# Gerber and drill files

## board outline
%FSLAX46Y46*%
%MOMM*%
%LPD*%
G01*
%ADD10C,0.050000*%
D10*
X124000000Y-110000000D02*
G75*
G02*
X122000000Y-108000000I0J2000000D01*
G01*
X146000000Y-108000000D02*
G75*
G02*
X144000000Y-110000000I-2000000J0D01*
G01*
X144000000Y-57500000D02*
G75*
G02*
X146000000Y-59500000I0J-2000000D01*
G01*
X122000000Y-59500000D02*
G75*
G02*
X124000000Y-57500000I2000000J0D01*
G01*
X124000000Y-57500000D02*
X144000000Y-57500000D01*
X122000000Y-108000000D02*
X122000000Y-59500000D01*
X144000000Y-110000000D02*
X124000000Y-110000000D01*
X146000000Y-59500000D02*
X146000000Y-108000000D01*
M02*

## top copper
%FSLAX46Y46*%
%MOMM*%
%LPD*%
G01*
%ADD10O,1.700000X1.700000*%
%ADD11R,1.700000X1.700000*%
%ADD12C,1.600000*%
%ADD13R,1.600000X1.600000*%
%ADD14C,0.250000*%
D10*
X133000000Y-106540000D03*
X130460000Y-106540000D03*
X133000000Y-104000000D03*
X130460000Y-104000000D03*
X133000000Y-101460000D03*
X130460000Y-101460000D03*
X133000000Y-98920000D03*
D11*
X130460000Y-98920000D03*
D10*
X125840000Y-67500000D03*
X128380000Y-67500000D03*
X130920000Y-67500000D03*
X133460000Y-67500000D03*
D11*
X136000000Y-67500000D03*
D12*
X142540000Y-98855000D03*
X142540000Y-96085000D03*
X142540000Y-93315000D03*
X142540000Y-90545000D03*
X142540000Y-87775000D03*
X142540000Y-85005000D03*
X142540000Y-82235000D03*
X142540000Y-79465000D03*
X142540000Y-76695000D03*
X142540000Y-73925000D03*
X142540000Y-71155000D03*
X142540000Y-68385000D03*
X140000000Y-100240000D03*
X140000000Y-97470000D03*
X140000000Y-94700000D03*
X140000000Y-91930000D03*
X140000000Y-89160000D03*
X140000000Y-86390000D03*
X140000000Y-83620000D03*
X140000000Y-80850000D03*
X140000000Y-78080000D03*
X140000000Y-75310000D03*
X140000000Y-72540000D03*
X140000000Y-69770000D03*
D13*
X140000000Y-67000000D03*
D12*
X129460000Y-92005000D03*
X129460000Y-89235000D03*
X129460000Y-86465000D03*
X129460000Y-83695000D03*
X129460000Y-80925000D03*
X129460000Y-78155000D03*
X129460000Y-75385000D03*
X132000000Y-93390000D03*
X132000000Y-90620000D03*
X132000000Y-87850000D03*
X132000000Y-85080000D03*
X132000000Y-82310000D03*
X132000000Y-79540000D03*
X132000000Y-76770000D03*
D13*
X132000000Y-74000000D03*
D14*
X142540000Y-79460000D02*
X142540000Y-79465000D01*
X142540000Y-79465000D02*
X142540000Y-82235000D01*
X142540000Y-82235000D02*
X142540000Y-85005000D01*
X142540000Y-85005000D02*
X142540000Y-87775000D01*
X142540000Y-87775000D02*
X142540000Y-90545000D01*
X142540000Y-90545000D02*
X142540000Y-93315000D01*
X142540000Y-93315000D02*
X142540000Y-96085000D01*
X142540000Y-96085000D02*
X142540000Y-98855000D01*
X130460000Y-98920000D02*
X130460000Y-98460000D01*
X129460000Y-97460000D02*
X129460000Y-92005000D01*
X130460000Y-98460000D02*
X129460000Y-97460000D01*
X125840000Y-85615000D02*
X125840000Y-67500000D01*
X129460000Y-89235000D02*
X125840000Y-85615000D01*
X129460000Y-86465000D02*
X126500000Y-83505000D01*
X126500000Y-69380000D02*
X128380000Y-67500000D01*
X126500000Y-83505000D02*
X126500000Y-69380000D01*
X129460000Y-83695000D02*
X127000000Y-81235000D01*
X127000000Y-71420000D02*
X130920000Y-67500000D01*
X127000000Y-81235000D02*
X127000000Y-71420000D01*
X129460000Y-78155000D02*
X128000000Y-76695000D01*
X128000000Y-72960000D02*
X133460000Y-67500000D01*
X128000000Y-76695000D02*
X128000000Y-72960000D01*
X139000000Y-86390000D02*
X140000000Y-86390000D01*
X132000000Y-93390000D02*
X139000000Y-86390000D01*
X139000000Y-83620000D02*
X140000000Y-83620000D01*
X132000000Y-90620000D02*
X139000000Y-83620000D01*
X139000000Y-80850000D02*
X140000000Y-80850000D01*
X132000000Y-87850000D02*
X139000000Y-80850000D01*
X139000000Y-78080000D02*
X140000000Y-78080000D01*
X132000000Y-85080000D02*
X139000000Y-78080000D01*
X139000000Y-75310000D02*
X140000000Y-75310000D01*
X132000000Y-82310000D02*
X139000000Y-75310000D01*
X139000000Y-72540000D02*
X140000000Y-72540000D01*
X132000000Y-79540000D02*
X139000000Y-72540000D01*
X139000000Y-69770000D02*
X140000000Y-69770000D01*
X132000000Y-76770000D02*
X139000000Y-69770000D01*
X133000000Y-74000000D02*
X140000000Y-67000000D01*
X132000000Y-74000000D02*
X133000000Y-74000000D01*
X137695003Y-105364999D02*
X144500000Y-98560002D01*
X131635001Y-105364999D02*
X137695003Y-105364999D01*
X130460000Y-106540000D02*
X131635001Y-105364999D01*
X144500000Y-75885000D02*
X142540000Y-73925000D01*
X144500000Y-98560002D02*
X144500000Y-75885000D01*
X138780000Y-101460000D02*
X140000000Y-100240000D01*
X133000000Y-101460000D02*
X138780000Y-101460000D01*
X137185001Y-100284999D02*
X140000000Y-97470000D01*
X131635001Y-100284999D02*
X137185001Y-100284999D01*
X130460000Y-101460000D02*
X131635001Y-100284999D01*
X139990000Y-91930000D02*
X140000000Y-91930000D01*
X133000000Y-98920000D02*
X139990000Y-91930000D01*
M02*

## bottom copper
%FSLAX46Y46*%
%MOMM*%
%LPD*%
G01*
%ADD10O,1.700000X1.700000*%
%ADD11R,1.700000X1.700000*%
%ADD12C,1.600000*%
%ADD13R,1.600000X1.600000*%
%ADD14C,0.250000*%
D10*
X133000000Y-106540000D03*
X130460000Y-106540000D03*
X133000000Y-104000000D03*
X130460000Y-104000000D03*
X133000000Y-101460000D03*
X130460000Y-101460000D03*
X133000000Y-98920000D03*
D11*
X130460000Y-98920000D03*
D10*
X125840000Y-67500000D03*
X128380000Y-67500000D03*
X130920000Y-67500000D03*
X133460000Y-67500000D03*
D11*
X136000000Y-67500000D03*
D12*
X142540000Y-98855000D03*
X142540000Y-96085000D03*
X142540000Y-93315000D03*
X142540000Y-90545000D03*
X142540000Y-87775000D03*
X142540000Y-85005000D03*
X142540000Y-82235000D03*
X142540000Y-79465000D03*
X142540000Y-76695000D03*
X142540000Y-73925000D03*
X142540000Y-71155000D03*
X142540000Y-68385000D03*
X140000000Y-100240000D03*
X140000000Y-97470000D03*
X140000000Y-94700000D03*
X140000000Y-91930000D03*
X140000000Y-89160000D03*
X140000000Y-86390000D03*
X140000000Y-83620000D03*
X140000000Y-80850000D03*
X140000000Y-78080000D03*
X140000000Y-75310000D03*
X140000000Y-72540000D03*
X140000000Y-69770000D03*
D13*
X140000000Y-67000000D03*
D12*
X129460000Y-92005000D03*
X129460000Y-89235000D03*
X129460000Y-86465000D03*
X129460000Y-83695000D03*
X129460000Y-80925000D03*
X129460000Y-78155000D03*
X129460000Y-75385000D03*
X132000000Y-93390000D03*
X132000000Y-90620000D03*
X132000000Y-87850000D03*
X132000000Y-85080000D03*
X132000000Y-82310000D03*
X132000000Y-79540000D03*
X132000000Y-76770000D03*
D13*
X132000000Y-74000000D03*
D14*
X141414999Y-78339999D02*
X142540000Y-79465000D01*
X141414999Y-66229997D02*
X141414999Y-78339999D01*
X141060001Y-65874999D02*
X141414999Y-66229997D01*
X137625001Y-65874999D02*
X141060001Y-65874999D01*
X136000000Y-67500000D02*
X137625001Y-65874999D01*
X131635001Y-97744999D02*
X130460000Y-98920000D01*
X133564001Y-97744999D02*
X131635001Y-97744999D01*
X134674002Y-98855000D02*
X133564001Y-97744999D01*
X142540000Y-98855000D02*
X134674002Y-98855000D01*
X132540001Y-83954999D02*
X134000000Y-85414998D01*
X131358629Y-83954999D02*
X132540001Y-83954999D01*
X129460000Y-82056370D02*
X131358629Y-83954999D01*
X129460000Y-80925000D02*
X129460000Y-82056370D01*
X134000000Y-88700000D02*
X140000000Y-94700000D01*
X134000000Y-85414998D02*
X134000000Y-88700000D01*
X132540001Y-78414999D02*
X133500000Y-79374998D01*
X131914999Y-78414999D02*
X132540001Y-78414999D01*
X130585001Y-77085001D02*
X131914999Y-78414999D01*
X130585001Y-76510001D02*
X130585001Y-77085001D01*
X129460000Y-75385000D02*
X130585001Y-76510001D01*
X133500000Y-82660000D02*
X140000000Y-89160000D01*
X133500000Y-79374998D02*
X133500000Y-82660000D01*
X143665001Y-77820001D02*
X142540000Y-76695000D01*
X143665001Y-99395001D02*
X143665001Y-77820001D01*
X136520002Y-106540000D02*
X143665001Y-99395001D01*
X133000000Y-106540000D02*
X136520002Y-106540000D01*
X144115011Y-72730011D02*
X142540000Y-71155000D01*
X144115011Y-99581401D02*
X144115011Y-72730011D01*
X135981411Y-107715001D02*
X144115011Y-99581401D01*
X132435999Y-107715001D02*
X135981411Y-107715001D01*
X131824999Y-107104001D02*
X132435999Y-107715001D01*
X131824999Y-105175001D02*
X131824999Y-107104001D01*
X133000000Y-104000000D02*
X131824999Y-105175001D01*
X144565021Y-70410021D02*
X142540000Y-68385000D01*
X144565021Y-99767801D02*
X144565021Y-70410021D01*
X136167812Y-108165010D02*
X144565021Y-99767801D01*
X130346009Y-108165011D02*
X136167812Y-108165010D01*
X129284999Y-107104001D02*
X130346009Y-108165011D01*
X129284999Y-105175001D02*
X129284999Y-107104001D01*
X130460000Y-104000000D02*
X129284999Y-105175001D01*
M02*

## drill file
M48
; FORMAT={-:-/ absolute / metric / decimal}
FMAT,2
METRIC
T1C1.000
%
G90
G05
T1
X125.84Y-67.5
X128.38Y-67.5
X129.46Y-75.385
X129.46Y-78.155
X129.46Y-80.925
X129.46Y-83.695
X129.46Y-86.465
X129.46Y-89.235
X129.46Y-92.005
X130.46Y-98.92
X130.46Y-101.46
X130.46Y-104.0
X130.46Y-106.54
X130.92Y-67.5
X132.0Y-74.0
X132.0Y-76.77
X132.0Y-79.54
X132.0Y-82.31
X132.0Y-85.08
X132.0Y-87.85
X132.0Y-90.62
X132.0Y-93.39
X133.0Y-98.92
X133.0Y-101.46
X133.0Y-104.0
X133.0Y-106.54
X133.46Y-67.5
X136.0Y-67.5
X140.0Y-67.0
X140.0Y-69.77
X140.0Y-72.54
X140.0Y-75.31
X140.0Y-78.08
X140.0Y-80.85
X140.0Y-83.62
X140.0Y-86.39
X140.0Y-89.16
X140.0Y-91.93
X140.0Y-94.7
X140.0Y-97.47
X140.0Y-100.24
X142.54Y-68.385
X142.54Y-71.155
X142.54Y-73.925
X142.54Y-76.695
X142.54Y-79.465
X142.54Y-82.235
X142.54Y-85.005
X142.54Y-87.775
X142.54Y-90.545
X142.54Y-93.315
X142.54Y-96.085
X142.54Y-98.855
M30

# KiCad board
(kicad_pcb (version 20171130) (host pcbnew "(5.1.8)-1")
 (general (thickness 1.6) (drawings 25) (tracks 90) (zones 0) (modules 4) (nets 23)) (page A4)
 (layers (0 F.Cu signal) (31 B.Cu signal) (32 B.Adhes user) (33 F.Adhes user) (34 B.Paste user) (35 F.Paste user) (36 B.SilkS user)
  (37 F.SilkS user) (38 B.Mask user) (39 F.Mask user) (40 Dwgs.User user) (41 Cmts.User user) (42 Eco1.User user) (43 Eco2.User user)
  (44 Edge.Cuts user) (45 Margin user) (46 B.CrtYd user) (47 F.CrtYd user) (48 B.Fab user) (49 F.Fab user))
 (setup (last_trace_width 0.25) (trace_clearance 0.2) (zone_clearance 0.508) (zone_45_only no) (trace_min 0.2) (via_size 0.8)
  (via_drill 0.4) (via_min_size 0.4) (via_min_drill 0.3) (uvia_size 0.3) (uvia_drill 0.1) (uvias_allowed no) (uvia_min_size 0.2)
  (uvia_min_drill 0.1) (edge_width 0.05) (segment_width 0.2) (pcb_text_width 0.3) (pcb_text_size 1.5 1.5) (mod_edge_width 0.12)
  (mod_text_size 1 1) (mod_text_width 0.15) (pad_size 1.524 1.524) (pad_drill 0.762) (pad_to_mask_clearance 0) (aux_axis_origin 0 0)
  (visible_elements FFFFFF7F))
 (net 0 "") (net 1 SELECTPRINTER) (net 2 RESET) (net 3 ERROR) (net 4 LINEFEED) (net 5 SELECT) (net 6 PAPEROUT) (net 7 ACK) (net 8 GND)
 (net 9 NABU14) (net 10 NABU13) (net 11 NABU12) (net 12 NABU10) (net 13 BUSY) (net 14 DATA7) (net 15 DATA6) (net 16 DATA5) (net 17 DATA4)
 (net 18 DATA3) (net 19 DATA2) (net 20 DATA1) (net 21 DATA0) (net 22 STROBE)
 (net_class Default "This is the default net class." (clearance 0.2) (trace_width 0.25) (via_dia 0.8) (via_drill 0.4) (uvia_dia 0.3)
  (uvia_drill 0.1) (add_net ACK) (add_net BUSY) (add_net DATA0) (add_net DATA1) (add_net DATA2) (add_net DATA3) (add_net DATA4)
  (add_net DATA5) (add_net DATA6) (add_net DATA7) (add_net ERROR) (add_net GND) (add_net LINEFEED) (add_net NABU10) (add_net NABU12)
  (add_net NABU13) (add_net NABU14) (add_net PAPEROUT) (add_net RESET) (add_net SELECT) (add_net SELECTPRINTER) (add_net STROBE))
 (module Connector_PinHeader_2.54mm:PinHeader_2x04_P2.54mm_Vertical (layer F.Cu) (at 130.46 98.92)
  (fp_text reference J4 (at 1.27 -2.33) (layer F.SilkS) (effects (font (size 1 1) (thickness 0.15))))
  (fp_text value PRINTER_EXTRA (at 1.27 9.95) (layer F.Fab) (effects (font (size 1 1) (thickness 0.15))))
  (pad 8 thru_hole oval (at 2.54 7.62) (size 1.7 1.7) (drill 1) (layers *.Cu *.Mask) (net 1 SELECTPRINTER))
  (pad 7 thru_hole oval (at 0 7.62) (size 1.7 1.7) (drill 1) (layers *.Cu *.Mask) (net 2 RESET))
  (pad 6 thru_hole oval (at 2.54 5.08) (size 1.7 1.7) (drill 1) (layers *.Cu *.Mask) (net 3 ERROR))
  (pad 5 thru_hole oval (at 0 5.08) (size 1.7 1.7) (drill 1) (layers *.Cu *.Mask) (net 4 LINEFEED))
  (pad 4 thru_hole oval (at 2.54 2.54) (size 1.7 1.7) (drill 1) (layers *.Cu *.Mask) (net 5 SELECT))
  (pad 3 thru_hole oval (at 0 2.54) (size 1.7 1.7) (drill 1) (layers *.Cu *.Mask) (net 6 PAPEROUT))
  (pad 2 thru_hole oval (at 2.54 0) (size 1.7 1.7) (drill 1) (layers *.Cu *.Mask) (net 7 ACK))
  (pad 1 thru_hole rect (at 0 0) (size 1.7 1.7) (drill 1) (layers *.Cu *.Mask) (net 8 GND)))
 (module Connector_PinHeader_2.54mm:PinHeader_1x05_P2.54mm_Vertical (layer F.Cu) (at 136 67.5 270)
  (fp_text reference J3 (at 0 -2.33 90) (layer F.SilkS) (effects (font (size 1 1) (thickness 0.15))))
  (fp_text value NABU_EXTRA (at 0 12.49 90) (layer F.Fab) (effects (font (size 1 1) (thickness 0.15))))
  (pad 5 thru_hole oval (at 0 10.16 270) (size 1.7 1.7) (drill 1) (layers *.Cu *.Mask) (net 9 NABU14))
  (pad 4 thru_hole oval (at 0 7.62 270) (size 1.7 1.7) (drill 1) (layers *.Cu *.Mask) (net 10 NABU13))
  (pad 3 thru_hole oval (at 0 5.08 270) (size 1.7 1.7) (drill 1) (layers *.Cu *.Mask) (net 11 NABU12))
  (pad 2 thru_hole oval (at 0 2.54 270) (size 1.7 1.7) (drill 1) (layers *.Cu *.Mask) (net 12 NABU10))
  (pad 1 thru_hole rect (at 0 0 270) (size 1.7 1.7) (drill 1) (layers *.Cu *.Mask) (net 8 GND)))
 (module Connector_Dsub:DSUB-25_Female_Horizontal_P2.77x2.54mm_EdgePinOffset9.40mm (layer F.Cu) (at 140 67 90)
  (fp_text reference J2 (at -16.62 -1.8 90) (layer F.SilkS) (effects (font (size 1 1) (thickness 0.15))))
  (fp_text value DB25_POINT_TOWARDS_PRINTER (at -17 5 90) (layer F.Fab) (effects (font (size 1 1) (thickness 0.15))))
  (pad 25 thru_hole circle (at -31.855 2.54 90) (size 1.6 1.6) (drill 1) (layers *.Cu *.Mask) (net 8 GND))
  (pad 24 thru_hole circle (at -29.085 2.54 90) (size 1.6 1.6) (drill 1) (layers *.Cu *.Mask) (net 8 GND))
  (pad 23 thru_hole circle (at -26.315 2.54 90) (size 1.6 1.6) (drill 1) (layers *.Cu *.Mask) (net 8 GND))
  (pad 22 thru_hole circle (at -23.545 2.54 90) (size 1.6 1.6) (drill 1) (layers *.Cu *.Mask) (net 8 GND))
  (pad 21 thru_hole circle (at -20.775 2.54 90) (size 1.6 1.6) (drill 1) (layers *.Cu *.Mask) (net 8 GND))
  (pad 20 thru_hole circle (at -18.005 2.54 90) (size 1.6 1.6) (drill 1) (layers *.Cu *.Mask) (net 8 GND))
  (pad 19 thru_hole circle (at -15.235 2.54 90) (size 1.6 1.6) (drill 1) (layers *.Cu *.Mask) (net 8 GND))
  (pad 18 thru_hole circle (at -12.465 2.54 90) (size 1.6 1.6) (drill 1) (layers *.Cu *.Mask) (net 8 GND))
  (pad 17 thru_hole circle (at -9.695 2.54 90) (size 1.6 1.6) (drill 1) (layers *.Cu *.Mask) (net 1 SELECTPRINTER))
  (pad 16 thru_hole circle (at -6.925 2.54 90) (size 1.6 1.6) (drill 1) (layers *.Cu *.Mask) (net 2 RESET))
  (pad 15 thru_hole circle (at -4.155 2.54 90) (size 1.6 1.6) (drill 1) (layers *.Cu *.Mask) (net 3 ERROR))
  (pad 14 thru_hole circle (at -1.385 2.54 90) (size 1.6 1.6) (drill 1) (layers *.Cu *.Mask) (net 4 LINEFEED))
  (pad 13 thru_hole circle (at -33.24 0 90) (size 1.6 1.6) (drill 1) (layers *.Cu *.Mask) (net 5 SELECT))
  (pad 12 thru_hole circle (at -30.47 0 90) (size 1.6 1.6) (drill 1) (layers *.Cu *.Mask) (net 6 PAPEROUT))
  (pad 11 thru_hole circle (at -27.7 0 90) (size 1.6 1.6) (drill 1) (layers *.Cu *.Mask) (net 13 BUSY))
  (pad 10 thru_hole circle (at -24.93 0 90) (size 1.6 1.6) (drill 1) (layers *.Cu *.Mask) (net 7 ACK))
  (pad 9 thru_hole circle (at -22.16 0 90) (size 1.6 1.6) (drill 1) (layers *.Cu *.Mask) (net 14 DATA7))
  (pad 8 thru_hole circle (at -19.39 0 90) (size 1.6 1.6) (drill 1) (layers *.Cu *.Mask) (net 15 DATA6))
  (pad 7 thru_hole circle (at -16.62 0 90) (size 1.6 1.6) (drill 1) (layers *.Cu *.Mask) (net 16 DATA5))
  (pad 6 thru_hole circle (at -13.85 0 90) (size 1.6 1.6) (drill 1) (layers *.Cu *.Mask) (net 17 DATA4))
  (pad 5 thru_hole circle (at -11.08 0 90) (size 1.6 1.6) (drill 1) (layers *.Cu *.Mask) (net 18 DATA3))
  (pad 4 thru_hole circle (at -8.31 0 90) (size 1.6 1.6) (drill 1) (layers *.Cu *.Mask) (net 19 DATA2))
  (pad 3 thru_hole circle (at -5.54 0 90) (size 1.6 1.6) (drill 1) (layers *.Cu *.Mask) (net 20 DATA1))
  (pad 2 thru_hole circle (at -2.77 0 90) (size 1.6 1.6) (drill 1) (layers *.Cu *.Mask) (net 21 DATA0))
  (pad 1 thru_hole rect (at 0 0 90) (size 1.6 1.6) (drill 1) (layers *.Cu *.Mask) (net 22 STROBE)))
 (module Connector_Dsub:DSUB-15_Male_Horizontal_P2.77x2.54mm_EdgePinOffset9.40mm (layer F.Cu) (at 132 74 270)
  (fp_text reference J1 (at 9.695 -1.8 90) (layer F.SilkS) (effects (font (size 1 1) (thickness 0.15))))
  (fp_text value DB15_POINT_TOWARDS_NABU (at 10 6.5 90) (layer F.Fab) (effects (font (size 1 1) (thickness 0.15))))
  (pad 15 thru_hole circle (at 18.005 2.54 270) (size 1.6 1.6) (drill 1) (layers *.Cu *.Mask) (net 8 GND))
  (pad 14 thru_hole circle (at 15.235 2.54 270) (size 1.6 1.6) (drill 1) (layers *.Cu *.Mask) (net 9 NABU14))
  (pad 13 thru_hole circle (at 12.465 2.54 270) (size 1.6 1.6) (drill 1) (layers *.Cu *.Mask) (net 10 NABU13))
  (pad 12 thru_hole circle (at 9.695 2.54 270) (size 1.6 1.6) (drill 1) (layers *.Cu *.Mask) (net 11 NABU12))
  (pad 11 thru_hole circle (at 6.925 2.54 270) (size 1.6 1.6) (drill 1) (layers *.Cu *.Mask) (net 13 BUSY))
  (pad 10 thru_hole circle (at 4.155 2.54 270) (size 1.6 1.6) (drill 1) (layers *.Cu *.Mask) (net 12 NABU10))
  (pad 9 thru_hole circle (at 1.385 2.54 270) (size 1.6 1.6) (drill 1) (layers *.Cu *.Mask) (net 14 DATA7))
  (pad 8 thru_hole circle (at 19.39 0 270) (size 1.6 1.6) (drill 1) (layers *.Cu *.Mask) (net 15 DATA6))
  (pad 7 thru_hole circle (at 16.62 0 270) (size 1.6 1.6) (drill 1) (layers *.Cu *.Mask) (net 16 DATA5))
  (pad 6 thru_hole circle (at 13.85 0 270) (size 1.6 1.6) (drill 1) (layers *.Cu *.Mask) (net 17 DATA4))
  (pad 5 thru_hole circle (at 11.08 0 270) (size 1.6 1.6) (drill 1) (layers *.Cu *.Mask) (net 18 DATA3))
  (pad 4 thru_hole circle (at 8.31 0 270) (size 1.6 1.6) (drill 1) (layers *.Cu *.Mask) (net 19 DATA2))
  (pad 3 thru_hole circle (at 5.54 0 270) (size 1.6 1.6) (drill 1) (layers *.Cu *.Mask) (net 20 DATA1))
  (pad 2 thru_hole circle (at 2.77 0 270) (size 1.6 1.6) (drill 1) (layers *.Cu *.Mask) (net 21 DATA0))
  (pad 1 thru_hole rect (at 0 0 270) (size 1.6 1.6) (drill 1) (layers *.Cu *.Mask) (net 22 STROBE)))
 (gr_arc (start 124 108) (end 122 108) (angle -90) (layer Edge.Cuts) (width 0.05))
 (gr_arc (start 144 108) (end 144 110) (angle -90) (layer Edge.Cuts) (width 0.05))
 (gr_arc (start 144 59.5) (end 146 59.5) (angle -90) (layer Edge.Cuts) (width 0.05))
 (gr_arc (start 124 59.5) (end 124 57.5) (angle -90) (layer Edge.Cuts) (width 0.05))
 (gr_line (start 124 57.5) (end 144 57.5) (layer Edge.Cuts) (width 0.05))
 (gr_line (start 122 108) (end 122 59.5) (layer Edge.Cuts) (width 0.05))
 (gr_line (start 144 110) (end 124 110) (layer Edge.Cuts) (width 0.05))
 (gr_line (start 146 59.5) (end 146 108) (layer Edge.Cuts) (width 0.05))
 (segment (start 142.54 79.46) (end 142.54 79.465) (width 0.25) (layer F.Cu) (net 8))
 (segment (start 142.54 79.465) (end 142.54 82.235) (width 0.25) (layer F.Cu) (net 8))
 (segment (start 142.54 82.235) (end 142.54 85.005) (width 0.25) (layer F.Cu) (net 8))
 (segment (start 142.54 85.005) (end 142.54 87.775) (width 0.25) (layer F.Cu) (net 8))
 (segment (start 142.54 87.775) (end 142.54 90.545) (width 0.25) (layer F.Cu) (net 8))
 (segment (start 142.54 90.545) (end 142.54 93.315) (width 0.25) (layer F.Cu) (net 8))
 (segment (start 142.54 93.315) (end 142.54 96.085) (width 0.25) (layer F.Cu) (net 8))
 (segment (start 142.54 96.085) (end 142.54 98.855) (width 0.25) (layer F.Cu) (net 8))
 (segment (start 130.46 98.92) (end 130.46 98.46) (width 0.25) (layer F.Cu) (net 8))
 (segment (start 129.46 97.46) (end 129.46 92.005) (width 0.25) (layer F.Cu) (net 8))
 (segment (start 130.46 98.46) (end 129.46 97.46) (width 0.25) (layer F.Cu) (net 8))
 (segment (start 141.414999 78.339999) (end 142.54 79.465) (width 0.25) (layer B.Cu) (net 8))
 (segment (start 141.414999 66.229997) (end 141.414999 78.339999) (width 0.25) (layer B.Cu) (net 8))
 (segment (start 141.060001 65.874999) (end 141.414999 66.229997) (width 0.25) (layer B.Cu) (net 8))
 (segment (start 137.625001 65.874999) (end 141.060001 65.874999) (width 0.25) (layer B.Cu) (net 8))
 (segment (start 136 67.5) (end 137.625001 65.874999) (width 0.25) (layer B.Cu) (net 8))
 (segment (start 131.635001 97.744999) (end 130.46 98.92) (width 0.25) (layer B.Cu) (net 8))
 (segment (start 133.564001 97.744999) (end 131.635001 97.744999) (width 0.25) (layer B.Cu) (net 8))
 (segment (start 134.674002 98.855) (end 133.564001 97.744999) (width 0.25) (layer B.Cu) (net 8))
 (segment (start 142.54 98.855) (end 134.674002 98.855) (width 0.25) (layer B.Cu) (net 8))
 (segment (start 125.84 85.615) (end 125.84 67.5) (width 0.25) (layer F.Cu) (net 9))
 (segment (start 129.46 89.235) (end 125.84 85.615) (width 0.25) (layer F.Cu) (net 9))
 (segment (start 129.46 86.465) (end 126.5 83.505) (width 0.25) (layer F.Cu) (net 10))
 (segment (start 126.5 69.38) (end 128.38 67.5) (width 0.25) (layer F.Cu) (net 10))
 (segment (start 126.5 83.505) (end 126.5 69.38) (width 0.25) (layer F.Cu) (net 10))
 (segment (start 129.46 83.695) (end 127 81.235) (width 0.25) (layer F.Cu) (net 11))
 (segment (start 127 71.42) (end 130.92 67.5) (width 0.25) (layer F.Cu) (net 11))
 (segment (start 127 81.235) (end 127 71.42) (width 0.25) (layer F.Cu) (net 11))
 (segment (start 132.540001 83.954999) (end 134 85.414998) (width 0.25) (layer B.Cu) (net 13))
 (segment (start 131.358629 83.954999) (end 132.540001 83.954999) (width 0.25) (layer B.Cu) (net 13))
 (segment (start 129.46 82.05637) (end 131.358629 83.954999) (width 0.25) (layer B.Cu) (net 13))
 (segment (start 129.46 80.925) (end 129.46 82.05637) (width 0.25) (layer B.Cu) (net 13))
 (segment (start 134 88.7) (end 140 94.7) (width 0.25) (layer B.Cu) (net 13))
 (segment (start 134 85.414998) (end 134 88.7) (width 0.25) (layer B.Cu) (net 13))
 (segment (start 129.46 78.155) (end 128 76.695) (width 0.25) (layer F.Cu) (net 12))
 (segment (start 128 72.96) (end 133.46 67.5) (width 0.25) (layer F.Cu) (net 12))
 (segment (start 128 76.695) (end 128 72.96) (width 0.25) (layer F.Cu) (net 12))
 (segment (start 132.540001 78.414999) (end 133.5 79.374998) (width 0.25) (layer B.Cu) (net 14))
 (segment (start 131.914999 78.414999) (end 132.540001 78.414999) (width 0.25) (layer B.Cu) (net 14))
 (segment (start 130.585001 77.085001) (end 131.914999 78.414999) (width 0.25) (layer B.Cu) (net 14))
 (segment (start 130.585001 76.510001) (end 130.585001 77.085001) (width 0.25) (layer B.Cu) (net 14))
 (segment (start 129.46 75.385) (end 130.585001 76.510001) (width 0.25) (layer B.Cu) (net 14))
 (segment (start 133.5 82.66) (end 140 89.16) (width 0.25) (layer B.Cu) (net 14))
 (segment (start 133.5 79.374998) (end 133.5 82.66) (width 0.25) (layer B.Cu) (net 14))
 (segment (start 139 86.39) (end 140 86.39) (width 0.25) (layer F.Cu) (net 15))
 (segment (start 132 93.39) (end 139 86.39) (width 0.25) (layer F.Cu) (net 15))
 (segment (start 139 83.62) (end 140 83.62) (width 0.25) (layer F.Cu) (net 16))
 (segment (start 132 90.62) (end 139 83.62) (width 0.25) (layer F.Cu) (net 16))
 (segment (start 139 80.85) (end 140 80.85) (width 0.25) (layer F.Cu) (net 17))
 (segment (start 132 87.85) (end 139 80.85) (width 0.25) (layer F.Cu) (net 17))
 (segment (start 139 78.08) (end 140 78.08) (width 0.25) (layer F.Cu) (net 18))
 (segment (start 132 85.08) (end 139 78.08) (width 0.25) (layer F.Cu) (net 18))
 (segment (start 139 75.31) (end 140 75.31) (width 0.25) (layer F.Cu) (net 19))
 (segment (start 132 82.31) (end 139 75.31) (width 0.25) (layer F.Cu) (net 19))
 (segment (start 139 72.54) (end 140 72.54) (width 0.25) (layer F.Cu) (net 20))
 (segment (start 132 79.54) (end 139 72.54) (width 0.25) (layer F.Cu) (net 20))
 (segment (start 139 69.77) (end 140 69.77) (width 0.25) (layer F.Cu) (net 21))
 (segment (start 132 76.77) (end 139 69.77) (width 0.25) (layer F.Cu) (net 21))
 (segment (start 133 74) (end 140 67) (width 0.25) (layer F.Cu) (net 22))
 (segment (start 132 74) (end 133 74) (width 0.25) (layer F.Cu) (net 22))
 (segment (start 143.665001 77.820001) (end 142.54 76.695) (width 0.25) (layer B.Cu) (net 1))
 (segment (start 143.665001 99.395001) (end 143.665001 77.820001) (width 0.25) (layer B.Cu) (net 1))
 (segment (start 136.520002 106.54) (end 143.665001 99.395001) (width 0.25) (layer B.Cu) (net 1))
 (segment (start 133 106.54) (end 136.520002 106.54) (width 0.25) (layer B.Cu) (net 1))
 (segment (start 137.695003 105.364999) (end 144.5 98.560002) (width 0.25) (layer F.Cu) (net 2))
 (segment (start 131.635001 105.364999) (end 137.695003 105.364999) (width 0.25) (layer F.Cu) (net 2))
 (segment (start 130.46 106.54) (end 131.635001 105.364999) (width 0.25) (layer F.Cu) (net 2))
 (segment (start 144.5 75.885) (end 142.54 73.925) (width 0.25) (layer F.Cu) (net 2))
 (segment (start 144.5 98.560002) (end 144.5 75.885) (width 0.25) (layer F.Cu) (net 2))
 (segment (start 144.115011 72.730011) (end 142.54 71.155) (width 0.25) (layer B.Cu) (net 3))
 (segment (start 144.115011 99.581401) (end 144.115011 72.730011) (width 0.25) (layer B.Cu) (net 3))
 (segment (start 135.981411 107.715001) (end 144.115011 99.581401) (width 0.25) (layer B.Cu) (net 3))
 (segment (start 132.435999 107.715001) (end 135.981411 107.715001) (width 0.25) (layer B.Cu) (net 3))
 (segment (start 131.824999 107.104001) (end 132.435999 107.715001) (width 0.25) (layer B.Cu) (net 3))
 (segment (start 131.824999 105.175001) (end 131.824999 107.104001) (width 0.25) (layer B.Cu) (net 3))
 (segment (start 133 104) (end 131.824999 105.175001) (width 0.25) (layer B.Cu) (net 3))
 (segment (start 144.565021 70.410021) (end 142.54 68.385) (width 0.25) (layer B.Cu) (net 4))
 (segment (start 144.565021 99.767801) (end 144.565021 70.410021) (width 0.25) (layer B.Cu) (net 4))
 (segment (start 136.167812 108.16501) (end 144.565021 99.767801) (width 0.25) (layer B.Cu) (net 4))
 (segment (start 130.346009 108.165011) (end 136.167812 108.16501) (width 0.25) (layer B.Cu) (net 4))
 (segment (start 129.284999 107.104001) (end 130.346009 108.165011) (width 0.25) (layer B.Cu) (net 4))
 (segment (start 129.284999 105.175001) (end 129.284999 107.104001) (width 0.25) (layer B.Cu) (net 4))
 (segment (start 130.46 104) (end 129.284999 105.175001) (width 0.25) (layer B.Cu) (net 4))
 (segment (start 138.78 101.46) (end 140 100.24) (width 0.25) (layer F.Cu) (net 5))
 (segment (start 133 101.46) (end 138.78 101.46) (width 0.25) (layer F.Cu) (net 5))
 (segment (start 137.185001 100.284999) (end 140 97.47) (width 0.25) (layer F.Cu) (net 6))
 (segment (start 131.635001 100.284999) (end 137.185001 100.284999) (width 0.25) (layer F.Cu) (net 6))
 (segment (start 130.46 101.46) (end 131.635001 100.284999) (width 0.25) (layer F.Cu) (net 6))
 (segment (start 139.99 91.93) (end 140 91.93) (width 0.25) (layer F.Cu) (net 7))
 (segment (start 133 98.92) (end 139.99 91.93) (width 0.25) (layer F.Cu) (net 7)))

